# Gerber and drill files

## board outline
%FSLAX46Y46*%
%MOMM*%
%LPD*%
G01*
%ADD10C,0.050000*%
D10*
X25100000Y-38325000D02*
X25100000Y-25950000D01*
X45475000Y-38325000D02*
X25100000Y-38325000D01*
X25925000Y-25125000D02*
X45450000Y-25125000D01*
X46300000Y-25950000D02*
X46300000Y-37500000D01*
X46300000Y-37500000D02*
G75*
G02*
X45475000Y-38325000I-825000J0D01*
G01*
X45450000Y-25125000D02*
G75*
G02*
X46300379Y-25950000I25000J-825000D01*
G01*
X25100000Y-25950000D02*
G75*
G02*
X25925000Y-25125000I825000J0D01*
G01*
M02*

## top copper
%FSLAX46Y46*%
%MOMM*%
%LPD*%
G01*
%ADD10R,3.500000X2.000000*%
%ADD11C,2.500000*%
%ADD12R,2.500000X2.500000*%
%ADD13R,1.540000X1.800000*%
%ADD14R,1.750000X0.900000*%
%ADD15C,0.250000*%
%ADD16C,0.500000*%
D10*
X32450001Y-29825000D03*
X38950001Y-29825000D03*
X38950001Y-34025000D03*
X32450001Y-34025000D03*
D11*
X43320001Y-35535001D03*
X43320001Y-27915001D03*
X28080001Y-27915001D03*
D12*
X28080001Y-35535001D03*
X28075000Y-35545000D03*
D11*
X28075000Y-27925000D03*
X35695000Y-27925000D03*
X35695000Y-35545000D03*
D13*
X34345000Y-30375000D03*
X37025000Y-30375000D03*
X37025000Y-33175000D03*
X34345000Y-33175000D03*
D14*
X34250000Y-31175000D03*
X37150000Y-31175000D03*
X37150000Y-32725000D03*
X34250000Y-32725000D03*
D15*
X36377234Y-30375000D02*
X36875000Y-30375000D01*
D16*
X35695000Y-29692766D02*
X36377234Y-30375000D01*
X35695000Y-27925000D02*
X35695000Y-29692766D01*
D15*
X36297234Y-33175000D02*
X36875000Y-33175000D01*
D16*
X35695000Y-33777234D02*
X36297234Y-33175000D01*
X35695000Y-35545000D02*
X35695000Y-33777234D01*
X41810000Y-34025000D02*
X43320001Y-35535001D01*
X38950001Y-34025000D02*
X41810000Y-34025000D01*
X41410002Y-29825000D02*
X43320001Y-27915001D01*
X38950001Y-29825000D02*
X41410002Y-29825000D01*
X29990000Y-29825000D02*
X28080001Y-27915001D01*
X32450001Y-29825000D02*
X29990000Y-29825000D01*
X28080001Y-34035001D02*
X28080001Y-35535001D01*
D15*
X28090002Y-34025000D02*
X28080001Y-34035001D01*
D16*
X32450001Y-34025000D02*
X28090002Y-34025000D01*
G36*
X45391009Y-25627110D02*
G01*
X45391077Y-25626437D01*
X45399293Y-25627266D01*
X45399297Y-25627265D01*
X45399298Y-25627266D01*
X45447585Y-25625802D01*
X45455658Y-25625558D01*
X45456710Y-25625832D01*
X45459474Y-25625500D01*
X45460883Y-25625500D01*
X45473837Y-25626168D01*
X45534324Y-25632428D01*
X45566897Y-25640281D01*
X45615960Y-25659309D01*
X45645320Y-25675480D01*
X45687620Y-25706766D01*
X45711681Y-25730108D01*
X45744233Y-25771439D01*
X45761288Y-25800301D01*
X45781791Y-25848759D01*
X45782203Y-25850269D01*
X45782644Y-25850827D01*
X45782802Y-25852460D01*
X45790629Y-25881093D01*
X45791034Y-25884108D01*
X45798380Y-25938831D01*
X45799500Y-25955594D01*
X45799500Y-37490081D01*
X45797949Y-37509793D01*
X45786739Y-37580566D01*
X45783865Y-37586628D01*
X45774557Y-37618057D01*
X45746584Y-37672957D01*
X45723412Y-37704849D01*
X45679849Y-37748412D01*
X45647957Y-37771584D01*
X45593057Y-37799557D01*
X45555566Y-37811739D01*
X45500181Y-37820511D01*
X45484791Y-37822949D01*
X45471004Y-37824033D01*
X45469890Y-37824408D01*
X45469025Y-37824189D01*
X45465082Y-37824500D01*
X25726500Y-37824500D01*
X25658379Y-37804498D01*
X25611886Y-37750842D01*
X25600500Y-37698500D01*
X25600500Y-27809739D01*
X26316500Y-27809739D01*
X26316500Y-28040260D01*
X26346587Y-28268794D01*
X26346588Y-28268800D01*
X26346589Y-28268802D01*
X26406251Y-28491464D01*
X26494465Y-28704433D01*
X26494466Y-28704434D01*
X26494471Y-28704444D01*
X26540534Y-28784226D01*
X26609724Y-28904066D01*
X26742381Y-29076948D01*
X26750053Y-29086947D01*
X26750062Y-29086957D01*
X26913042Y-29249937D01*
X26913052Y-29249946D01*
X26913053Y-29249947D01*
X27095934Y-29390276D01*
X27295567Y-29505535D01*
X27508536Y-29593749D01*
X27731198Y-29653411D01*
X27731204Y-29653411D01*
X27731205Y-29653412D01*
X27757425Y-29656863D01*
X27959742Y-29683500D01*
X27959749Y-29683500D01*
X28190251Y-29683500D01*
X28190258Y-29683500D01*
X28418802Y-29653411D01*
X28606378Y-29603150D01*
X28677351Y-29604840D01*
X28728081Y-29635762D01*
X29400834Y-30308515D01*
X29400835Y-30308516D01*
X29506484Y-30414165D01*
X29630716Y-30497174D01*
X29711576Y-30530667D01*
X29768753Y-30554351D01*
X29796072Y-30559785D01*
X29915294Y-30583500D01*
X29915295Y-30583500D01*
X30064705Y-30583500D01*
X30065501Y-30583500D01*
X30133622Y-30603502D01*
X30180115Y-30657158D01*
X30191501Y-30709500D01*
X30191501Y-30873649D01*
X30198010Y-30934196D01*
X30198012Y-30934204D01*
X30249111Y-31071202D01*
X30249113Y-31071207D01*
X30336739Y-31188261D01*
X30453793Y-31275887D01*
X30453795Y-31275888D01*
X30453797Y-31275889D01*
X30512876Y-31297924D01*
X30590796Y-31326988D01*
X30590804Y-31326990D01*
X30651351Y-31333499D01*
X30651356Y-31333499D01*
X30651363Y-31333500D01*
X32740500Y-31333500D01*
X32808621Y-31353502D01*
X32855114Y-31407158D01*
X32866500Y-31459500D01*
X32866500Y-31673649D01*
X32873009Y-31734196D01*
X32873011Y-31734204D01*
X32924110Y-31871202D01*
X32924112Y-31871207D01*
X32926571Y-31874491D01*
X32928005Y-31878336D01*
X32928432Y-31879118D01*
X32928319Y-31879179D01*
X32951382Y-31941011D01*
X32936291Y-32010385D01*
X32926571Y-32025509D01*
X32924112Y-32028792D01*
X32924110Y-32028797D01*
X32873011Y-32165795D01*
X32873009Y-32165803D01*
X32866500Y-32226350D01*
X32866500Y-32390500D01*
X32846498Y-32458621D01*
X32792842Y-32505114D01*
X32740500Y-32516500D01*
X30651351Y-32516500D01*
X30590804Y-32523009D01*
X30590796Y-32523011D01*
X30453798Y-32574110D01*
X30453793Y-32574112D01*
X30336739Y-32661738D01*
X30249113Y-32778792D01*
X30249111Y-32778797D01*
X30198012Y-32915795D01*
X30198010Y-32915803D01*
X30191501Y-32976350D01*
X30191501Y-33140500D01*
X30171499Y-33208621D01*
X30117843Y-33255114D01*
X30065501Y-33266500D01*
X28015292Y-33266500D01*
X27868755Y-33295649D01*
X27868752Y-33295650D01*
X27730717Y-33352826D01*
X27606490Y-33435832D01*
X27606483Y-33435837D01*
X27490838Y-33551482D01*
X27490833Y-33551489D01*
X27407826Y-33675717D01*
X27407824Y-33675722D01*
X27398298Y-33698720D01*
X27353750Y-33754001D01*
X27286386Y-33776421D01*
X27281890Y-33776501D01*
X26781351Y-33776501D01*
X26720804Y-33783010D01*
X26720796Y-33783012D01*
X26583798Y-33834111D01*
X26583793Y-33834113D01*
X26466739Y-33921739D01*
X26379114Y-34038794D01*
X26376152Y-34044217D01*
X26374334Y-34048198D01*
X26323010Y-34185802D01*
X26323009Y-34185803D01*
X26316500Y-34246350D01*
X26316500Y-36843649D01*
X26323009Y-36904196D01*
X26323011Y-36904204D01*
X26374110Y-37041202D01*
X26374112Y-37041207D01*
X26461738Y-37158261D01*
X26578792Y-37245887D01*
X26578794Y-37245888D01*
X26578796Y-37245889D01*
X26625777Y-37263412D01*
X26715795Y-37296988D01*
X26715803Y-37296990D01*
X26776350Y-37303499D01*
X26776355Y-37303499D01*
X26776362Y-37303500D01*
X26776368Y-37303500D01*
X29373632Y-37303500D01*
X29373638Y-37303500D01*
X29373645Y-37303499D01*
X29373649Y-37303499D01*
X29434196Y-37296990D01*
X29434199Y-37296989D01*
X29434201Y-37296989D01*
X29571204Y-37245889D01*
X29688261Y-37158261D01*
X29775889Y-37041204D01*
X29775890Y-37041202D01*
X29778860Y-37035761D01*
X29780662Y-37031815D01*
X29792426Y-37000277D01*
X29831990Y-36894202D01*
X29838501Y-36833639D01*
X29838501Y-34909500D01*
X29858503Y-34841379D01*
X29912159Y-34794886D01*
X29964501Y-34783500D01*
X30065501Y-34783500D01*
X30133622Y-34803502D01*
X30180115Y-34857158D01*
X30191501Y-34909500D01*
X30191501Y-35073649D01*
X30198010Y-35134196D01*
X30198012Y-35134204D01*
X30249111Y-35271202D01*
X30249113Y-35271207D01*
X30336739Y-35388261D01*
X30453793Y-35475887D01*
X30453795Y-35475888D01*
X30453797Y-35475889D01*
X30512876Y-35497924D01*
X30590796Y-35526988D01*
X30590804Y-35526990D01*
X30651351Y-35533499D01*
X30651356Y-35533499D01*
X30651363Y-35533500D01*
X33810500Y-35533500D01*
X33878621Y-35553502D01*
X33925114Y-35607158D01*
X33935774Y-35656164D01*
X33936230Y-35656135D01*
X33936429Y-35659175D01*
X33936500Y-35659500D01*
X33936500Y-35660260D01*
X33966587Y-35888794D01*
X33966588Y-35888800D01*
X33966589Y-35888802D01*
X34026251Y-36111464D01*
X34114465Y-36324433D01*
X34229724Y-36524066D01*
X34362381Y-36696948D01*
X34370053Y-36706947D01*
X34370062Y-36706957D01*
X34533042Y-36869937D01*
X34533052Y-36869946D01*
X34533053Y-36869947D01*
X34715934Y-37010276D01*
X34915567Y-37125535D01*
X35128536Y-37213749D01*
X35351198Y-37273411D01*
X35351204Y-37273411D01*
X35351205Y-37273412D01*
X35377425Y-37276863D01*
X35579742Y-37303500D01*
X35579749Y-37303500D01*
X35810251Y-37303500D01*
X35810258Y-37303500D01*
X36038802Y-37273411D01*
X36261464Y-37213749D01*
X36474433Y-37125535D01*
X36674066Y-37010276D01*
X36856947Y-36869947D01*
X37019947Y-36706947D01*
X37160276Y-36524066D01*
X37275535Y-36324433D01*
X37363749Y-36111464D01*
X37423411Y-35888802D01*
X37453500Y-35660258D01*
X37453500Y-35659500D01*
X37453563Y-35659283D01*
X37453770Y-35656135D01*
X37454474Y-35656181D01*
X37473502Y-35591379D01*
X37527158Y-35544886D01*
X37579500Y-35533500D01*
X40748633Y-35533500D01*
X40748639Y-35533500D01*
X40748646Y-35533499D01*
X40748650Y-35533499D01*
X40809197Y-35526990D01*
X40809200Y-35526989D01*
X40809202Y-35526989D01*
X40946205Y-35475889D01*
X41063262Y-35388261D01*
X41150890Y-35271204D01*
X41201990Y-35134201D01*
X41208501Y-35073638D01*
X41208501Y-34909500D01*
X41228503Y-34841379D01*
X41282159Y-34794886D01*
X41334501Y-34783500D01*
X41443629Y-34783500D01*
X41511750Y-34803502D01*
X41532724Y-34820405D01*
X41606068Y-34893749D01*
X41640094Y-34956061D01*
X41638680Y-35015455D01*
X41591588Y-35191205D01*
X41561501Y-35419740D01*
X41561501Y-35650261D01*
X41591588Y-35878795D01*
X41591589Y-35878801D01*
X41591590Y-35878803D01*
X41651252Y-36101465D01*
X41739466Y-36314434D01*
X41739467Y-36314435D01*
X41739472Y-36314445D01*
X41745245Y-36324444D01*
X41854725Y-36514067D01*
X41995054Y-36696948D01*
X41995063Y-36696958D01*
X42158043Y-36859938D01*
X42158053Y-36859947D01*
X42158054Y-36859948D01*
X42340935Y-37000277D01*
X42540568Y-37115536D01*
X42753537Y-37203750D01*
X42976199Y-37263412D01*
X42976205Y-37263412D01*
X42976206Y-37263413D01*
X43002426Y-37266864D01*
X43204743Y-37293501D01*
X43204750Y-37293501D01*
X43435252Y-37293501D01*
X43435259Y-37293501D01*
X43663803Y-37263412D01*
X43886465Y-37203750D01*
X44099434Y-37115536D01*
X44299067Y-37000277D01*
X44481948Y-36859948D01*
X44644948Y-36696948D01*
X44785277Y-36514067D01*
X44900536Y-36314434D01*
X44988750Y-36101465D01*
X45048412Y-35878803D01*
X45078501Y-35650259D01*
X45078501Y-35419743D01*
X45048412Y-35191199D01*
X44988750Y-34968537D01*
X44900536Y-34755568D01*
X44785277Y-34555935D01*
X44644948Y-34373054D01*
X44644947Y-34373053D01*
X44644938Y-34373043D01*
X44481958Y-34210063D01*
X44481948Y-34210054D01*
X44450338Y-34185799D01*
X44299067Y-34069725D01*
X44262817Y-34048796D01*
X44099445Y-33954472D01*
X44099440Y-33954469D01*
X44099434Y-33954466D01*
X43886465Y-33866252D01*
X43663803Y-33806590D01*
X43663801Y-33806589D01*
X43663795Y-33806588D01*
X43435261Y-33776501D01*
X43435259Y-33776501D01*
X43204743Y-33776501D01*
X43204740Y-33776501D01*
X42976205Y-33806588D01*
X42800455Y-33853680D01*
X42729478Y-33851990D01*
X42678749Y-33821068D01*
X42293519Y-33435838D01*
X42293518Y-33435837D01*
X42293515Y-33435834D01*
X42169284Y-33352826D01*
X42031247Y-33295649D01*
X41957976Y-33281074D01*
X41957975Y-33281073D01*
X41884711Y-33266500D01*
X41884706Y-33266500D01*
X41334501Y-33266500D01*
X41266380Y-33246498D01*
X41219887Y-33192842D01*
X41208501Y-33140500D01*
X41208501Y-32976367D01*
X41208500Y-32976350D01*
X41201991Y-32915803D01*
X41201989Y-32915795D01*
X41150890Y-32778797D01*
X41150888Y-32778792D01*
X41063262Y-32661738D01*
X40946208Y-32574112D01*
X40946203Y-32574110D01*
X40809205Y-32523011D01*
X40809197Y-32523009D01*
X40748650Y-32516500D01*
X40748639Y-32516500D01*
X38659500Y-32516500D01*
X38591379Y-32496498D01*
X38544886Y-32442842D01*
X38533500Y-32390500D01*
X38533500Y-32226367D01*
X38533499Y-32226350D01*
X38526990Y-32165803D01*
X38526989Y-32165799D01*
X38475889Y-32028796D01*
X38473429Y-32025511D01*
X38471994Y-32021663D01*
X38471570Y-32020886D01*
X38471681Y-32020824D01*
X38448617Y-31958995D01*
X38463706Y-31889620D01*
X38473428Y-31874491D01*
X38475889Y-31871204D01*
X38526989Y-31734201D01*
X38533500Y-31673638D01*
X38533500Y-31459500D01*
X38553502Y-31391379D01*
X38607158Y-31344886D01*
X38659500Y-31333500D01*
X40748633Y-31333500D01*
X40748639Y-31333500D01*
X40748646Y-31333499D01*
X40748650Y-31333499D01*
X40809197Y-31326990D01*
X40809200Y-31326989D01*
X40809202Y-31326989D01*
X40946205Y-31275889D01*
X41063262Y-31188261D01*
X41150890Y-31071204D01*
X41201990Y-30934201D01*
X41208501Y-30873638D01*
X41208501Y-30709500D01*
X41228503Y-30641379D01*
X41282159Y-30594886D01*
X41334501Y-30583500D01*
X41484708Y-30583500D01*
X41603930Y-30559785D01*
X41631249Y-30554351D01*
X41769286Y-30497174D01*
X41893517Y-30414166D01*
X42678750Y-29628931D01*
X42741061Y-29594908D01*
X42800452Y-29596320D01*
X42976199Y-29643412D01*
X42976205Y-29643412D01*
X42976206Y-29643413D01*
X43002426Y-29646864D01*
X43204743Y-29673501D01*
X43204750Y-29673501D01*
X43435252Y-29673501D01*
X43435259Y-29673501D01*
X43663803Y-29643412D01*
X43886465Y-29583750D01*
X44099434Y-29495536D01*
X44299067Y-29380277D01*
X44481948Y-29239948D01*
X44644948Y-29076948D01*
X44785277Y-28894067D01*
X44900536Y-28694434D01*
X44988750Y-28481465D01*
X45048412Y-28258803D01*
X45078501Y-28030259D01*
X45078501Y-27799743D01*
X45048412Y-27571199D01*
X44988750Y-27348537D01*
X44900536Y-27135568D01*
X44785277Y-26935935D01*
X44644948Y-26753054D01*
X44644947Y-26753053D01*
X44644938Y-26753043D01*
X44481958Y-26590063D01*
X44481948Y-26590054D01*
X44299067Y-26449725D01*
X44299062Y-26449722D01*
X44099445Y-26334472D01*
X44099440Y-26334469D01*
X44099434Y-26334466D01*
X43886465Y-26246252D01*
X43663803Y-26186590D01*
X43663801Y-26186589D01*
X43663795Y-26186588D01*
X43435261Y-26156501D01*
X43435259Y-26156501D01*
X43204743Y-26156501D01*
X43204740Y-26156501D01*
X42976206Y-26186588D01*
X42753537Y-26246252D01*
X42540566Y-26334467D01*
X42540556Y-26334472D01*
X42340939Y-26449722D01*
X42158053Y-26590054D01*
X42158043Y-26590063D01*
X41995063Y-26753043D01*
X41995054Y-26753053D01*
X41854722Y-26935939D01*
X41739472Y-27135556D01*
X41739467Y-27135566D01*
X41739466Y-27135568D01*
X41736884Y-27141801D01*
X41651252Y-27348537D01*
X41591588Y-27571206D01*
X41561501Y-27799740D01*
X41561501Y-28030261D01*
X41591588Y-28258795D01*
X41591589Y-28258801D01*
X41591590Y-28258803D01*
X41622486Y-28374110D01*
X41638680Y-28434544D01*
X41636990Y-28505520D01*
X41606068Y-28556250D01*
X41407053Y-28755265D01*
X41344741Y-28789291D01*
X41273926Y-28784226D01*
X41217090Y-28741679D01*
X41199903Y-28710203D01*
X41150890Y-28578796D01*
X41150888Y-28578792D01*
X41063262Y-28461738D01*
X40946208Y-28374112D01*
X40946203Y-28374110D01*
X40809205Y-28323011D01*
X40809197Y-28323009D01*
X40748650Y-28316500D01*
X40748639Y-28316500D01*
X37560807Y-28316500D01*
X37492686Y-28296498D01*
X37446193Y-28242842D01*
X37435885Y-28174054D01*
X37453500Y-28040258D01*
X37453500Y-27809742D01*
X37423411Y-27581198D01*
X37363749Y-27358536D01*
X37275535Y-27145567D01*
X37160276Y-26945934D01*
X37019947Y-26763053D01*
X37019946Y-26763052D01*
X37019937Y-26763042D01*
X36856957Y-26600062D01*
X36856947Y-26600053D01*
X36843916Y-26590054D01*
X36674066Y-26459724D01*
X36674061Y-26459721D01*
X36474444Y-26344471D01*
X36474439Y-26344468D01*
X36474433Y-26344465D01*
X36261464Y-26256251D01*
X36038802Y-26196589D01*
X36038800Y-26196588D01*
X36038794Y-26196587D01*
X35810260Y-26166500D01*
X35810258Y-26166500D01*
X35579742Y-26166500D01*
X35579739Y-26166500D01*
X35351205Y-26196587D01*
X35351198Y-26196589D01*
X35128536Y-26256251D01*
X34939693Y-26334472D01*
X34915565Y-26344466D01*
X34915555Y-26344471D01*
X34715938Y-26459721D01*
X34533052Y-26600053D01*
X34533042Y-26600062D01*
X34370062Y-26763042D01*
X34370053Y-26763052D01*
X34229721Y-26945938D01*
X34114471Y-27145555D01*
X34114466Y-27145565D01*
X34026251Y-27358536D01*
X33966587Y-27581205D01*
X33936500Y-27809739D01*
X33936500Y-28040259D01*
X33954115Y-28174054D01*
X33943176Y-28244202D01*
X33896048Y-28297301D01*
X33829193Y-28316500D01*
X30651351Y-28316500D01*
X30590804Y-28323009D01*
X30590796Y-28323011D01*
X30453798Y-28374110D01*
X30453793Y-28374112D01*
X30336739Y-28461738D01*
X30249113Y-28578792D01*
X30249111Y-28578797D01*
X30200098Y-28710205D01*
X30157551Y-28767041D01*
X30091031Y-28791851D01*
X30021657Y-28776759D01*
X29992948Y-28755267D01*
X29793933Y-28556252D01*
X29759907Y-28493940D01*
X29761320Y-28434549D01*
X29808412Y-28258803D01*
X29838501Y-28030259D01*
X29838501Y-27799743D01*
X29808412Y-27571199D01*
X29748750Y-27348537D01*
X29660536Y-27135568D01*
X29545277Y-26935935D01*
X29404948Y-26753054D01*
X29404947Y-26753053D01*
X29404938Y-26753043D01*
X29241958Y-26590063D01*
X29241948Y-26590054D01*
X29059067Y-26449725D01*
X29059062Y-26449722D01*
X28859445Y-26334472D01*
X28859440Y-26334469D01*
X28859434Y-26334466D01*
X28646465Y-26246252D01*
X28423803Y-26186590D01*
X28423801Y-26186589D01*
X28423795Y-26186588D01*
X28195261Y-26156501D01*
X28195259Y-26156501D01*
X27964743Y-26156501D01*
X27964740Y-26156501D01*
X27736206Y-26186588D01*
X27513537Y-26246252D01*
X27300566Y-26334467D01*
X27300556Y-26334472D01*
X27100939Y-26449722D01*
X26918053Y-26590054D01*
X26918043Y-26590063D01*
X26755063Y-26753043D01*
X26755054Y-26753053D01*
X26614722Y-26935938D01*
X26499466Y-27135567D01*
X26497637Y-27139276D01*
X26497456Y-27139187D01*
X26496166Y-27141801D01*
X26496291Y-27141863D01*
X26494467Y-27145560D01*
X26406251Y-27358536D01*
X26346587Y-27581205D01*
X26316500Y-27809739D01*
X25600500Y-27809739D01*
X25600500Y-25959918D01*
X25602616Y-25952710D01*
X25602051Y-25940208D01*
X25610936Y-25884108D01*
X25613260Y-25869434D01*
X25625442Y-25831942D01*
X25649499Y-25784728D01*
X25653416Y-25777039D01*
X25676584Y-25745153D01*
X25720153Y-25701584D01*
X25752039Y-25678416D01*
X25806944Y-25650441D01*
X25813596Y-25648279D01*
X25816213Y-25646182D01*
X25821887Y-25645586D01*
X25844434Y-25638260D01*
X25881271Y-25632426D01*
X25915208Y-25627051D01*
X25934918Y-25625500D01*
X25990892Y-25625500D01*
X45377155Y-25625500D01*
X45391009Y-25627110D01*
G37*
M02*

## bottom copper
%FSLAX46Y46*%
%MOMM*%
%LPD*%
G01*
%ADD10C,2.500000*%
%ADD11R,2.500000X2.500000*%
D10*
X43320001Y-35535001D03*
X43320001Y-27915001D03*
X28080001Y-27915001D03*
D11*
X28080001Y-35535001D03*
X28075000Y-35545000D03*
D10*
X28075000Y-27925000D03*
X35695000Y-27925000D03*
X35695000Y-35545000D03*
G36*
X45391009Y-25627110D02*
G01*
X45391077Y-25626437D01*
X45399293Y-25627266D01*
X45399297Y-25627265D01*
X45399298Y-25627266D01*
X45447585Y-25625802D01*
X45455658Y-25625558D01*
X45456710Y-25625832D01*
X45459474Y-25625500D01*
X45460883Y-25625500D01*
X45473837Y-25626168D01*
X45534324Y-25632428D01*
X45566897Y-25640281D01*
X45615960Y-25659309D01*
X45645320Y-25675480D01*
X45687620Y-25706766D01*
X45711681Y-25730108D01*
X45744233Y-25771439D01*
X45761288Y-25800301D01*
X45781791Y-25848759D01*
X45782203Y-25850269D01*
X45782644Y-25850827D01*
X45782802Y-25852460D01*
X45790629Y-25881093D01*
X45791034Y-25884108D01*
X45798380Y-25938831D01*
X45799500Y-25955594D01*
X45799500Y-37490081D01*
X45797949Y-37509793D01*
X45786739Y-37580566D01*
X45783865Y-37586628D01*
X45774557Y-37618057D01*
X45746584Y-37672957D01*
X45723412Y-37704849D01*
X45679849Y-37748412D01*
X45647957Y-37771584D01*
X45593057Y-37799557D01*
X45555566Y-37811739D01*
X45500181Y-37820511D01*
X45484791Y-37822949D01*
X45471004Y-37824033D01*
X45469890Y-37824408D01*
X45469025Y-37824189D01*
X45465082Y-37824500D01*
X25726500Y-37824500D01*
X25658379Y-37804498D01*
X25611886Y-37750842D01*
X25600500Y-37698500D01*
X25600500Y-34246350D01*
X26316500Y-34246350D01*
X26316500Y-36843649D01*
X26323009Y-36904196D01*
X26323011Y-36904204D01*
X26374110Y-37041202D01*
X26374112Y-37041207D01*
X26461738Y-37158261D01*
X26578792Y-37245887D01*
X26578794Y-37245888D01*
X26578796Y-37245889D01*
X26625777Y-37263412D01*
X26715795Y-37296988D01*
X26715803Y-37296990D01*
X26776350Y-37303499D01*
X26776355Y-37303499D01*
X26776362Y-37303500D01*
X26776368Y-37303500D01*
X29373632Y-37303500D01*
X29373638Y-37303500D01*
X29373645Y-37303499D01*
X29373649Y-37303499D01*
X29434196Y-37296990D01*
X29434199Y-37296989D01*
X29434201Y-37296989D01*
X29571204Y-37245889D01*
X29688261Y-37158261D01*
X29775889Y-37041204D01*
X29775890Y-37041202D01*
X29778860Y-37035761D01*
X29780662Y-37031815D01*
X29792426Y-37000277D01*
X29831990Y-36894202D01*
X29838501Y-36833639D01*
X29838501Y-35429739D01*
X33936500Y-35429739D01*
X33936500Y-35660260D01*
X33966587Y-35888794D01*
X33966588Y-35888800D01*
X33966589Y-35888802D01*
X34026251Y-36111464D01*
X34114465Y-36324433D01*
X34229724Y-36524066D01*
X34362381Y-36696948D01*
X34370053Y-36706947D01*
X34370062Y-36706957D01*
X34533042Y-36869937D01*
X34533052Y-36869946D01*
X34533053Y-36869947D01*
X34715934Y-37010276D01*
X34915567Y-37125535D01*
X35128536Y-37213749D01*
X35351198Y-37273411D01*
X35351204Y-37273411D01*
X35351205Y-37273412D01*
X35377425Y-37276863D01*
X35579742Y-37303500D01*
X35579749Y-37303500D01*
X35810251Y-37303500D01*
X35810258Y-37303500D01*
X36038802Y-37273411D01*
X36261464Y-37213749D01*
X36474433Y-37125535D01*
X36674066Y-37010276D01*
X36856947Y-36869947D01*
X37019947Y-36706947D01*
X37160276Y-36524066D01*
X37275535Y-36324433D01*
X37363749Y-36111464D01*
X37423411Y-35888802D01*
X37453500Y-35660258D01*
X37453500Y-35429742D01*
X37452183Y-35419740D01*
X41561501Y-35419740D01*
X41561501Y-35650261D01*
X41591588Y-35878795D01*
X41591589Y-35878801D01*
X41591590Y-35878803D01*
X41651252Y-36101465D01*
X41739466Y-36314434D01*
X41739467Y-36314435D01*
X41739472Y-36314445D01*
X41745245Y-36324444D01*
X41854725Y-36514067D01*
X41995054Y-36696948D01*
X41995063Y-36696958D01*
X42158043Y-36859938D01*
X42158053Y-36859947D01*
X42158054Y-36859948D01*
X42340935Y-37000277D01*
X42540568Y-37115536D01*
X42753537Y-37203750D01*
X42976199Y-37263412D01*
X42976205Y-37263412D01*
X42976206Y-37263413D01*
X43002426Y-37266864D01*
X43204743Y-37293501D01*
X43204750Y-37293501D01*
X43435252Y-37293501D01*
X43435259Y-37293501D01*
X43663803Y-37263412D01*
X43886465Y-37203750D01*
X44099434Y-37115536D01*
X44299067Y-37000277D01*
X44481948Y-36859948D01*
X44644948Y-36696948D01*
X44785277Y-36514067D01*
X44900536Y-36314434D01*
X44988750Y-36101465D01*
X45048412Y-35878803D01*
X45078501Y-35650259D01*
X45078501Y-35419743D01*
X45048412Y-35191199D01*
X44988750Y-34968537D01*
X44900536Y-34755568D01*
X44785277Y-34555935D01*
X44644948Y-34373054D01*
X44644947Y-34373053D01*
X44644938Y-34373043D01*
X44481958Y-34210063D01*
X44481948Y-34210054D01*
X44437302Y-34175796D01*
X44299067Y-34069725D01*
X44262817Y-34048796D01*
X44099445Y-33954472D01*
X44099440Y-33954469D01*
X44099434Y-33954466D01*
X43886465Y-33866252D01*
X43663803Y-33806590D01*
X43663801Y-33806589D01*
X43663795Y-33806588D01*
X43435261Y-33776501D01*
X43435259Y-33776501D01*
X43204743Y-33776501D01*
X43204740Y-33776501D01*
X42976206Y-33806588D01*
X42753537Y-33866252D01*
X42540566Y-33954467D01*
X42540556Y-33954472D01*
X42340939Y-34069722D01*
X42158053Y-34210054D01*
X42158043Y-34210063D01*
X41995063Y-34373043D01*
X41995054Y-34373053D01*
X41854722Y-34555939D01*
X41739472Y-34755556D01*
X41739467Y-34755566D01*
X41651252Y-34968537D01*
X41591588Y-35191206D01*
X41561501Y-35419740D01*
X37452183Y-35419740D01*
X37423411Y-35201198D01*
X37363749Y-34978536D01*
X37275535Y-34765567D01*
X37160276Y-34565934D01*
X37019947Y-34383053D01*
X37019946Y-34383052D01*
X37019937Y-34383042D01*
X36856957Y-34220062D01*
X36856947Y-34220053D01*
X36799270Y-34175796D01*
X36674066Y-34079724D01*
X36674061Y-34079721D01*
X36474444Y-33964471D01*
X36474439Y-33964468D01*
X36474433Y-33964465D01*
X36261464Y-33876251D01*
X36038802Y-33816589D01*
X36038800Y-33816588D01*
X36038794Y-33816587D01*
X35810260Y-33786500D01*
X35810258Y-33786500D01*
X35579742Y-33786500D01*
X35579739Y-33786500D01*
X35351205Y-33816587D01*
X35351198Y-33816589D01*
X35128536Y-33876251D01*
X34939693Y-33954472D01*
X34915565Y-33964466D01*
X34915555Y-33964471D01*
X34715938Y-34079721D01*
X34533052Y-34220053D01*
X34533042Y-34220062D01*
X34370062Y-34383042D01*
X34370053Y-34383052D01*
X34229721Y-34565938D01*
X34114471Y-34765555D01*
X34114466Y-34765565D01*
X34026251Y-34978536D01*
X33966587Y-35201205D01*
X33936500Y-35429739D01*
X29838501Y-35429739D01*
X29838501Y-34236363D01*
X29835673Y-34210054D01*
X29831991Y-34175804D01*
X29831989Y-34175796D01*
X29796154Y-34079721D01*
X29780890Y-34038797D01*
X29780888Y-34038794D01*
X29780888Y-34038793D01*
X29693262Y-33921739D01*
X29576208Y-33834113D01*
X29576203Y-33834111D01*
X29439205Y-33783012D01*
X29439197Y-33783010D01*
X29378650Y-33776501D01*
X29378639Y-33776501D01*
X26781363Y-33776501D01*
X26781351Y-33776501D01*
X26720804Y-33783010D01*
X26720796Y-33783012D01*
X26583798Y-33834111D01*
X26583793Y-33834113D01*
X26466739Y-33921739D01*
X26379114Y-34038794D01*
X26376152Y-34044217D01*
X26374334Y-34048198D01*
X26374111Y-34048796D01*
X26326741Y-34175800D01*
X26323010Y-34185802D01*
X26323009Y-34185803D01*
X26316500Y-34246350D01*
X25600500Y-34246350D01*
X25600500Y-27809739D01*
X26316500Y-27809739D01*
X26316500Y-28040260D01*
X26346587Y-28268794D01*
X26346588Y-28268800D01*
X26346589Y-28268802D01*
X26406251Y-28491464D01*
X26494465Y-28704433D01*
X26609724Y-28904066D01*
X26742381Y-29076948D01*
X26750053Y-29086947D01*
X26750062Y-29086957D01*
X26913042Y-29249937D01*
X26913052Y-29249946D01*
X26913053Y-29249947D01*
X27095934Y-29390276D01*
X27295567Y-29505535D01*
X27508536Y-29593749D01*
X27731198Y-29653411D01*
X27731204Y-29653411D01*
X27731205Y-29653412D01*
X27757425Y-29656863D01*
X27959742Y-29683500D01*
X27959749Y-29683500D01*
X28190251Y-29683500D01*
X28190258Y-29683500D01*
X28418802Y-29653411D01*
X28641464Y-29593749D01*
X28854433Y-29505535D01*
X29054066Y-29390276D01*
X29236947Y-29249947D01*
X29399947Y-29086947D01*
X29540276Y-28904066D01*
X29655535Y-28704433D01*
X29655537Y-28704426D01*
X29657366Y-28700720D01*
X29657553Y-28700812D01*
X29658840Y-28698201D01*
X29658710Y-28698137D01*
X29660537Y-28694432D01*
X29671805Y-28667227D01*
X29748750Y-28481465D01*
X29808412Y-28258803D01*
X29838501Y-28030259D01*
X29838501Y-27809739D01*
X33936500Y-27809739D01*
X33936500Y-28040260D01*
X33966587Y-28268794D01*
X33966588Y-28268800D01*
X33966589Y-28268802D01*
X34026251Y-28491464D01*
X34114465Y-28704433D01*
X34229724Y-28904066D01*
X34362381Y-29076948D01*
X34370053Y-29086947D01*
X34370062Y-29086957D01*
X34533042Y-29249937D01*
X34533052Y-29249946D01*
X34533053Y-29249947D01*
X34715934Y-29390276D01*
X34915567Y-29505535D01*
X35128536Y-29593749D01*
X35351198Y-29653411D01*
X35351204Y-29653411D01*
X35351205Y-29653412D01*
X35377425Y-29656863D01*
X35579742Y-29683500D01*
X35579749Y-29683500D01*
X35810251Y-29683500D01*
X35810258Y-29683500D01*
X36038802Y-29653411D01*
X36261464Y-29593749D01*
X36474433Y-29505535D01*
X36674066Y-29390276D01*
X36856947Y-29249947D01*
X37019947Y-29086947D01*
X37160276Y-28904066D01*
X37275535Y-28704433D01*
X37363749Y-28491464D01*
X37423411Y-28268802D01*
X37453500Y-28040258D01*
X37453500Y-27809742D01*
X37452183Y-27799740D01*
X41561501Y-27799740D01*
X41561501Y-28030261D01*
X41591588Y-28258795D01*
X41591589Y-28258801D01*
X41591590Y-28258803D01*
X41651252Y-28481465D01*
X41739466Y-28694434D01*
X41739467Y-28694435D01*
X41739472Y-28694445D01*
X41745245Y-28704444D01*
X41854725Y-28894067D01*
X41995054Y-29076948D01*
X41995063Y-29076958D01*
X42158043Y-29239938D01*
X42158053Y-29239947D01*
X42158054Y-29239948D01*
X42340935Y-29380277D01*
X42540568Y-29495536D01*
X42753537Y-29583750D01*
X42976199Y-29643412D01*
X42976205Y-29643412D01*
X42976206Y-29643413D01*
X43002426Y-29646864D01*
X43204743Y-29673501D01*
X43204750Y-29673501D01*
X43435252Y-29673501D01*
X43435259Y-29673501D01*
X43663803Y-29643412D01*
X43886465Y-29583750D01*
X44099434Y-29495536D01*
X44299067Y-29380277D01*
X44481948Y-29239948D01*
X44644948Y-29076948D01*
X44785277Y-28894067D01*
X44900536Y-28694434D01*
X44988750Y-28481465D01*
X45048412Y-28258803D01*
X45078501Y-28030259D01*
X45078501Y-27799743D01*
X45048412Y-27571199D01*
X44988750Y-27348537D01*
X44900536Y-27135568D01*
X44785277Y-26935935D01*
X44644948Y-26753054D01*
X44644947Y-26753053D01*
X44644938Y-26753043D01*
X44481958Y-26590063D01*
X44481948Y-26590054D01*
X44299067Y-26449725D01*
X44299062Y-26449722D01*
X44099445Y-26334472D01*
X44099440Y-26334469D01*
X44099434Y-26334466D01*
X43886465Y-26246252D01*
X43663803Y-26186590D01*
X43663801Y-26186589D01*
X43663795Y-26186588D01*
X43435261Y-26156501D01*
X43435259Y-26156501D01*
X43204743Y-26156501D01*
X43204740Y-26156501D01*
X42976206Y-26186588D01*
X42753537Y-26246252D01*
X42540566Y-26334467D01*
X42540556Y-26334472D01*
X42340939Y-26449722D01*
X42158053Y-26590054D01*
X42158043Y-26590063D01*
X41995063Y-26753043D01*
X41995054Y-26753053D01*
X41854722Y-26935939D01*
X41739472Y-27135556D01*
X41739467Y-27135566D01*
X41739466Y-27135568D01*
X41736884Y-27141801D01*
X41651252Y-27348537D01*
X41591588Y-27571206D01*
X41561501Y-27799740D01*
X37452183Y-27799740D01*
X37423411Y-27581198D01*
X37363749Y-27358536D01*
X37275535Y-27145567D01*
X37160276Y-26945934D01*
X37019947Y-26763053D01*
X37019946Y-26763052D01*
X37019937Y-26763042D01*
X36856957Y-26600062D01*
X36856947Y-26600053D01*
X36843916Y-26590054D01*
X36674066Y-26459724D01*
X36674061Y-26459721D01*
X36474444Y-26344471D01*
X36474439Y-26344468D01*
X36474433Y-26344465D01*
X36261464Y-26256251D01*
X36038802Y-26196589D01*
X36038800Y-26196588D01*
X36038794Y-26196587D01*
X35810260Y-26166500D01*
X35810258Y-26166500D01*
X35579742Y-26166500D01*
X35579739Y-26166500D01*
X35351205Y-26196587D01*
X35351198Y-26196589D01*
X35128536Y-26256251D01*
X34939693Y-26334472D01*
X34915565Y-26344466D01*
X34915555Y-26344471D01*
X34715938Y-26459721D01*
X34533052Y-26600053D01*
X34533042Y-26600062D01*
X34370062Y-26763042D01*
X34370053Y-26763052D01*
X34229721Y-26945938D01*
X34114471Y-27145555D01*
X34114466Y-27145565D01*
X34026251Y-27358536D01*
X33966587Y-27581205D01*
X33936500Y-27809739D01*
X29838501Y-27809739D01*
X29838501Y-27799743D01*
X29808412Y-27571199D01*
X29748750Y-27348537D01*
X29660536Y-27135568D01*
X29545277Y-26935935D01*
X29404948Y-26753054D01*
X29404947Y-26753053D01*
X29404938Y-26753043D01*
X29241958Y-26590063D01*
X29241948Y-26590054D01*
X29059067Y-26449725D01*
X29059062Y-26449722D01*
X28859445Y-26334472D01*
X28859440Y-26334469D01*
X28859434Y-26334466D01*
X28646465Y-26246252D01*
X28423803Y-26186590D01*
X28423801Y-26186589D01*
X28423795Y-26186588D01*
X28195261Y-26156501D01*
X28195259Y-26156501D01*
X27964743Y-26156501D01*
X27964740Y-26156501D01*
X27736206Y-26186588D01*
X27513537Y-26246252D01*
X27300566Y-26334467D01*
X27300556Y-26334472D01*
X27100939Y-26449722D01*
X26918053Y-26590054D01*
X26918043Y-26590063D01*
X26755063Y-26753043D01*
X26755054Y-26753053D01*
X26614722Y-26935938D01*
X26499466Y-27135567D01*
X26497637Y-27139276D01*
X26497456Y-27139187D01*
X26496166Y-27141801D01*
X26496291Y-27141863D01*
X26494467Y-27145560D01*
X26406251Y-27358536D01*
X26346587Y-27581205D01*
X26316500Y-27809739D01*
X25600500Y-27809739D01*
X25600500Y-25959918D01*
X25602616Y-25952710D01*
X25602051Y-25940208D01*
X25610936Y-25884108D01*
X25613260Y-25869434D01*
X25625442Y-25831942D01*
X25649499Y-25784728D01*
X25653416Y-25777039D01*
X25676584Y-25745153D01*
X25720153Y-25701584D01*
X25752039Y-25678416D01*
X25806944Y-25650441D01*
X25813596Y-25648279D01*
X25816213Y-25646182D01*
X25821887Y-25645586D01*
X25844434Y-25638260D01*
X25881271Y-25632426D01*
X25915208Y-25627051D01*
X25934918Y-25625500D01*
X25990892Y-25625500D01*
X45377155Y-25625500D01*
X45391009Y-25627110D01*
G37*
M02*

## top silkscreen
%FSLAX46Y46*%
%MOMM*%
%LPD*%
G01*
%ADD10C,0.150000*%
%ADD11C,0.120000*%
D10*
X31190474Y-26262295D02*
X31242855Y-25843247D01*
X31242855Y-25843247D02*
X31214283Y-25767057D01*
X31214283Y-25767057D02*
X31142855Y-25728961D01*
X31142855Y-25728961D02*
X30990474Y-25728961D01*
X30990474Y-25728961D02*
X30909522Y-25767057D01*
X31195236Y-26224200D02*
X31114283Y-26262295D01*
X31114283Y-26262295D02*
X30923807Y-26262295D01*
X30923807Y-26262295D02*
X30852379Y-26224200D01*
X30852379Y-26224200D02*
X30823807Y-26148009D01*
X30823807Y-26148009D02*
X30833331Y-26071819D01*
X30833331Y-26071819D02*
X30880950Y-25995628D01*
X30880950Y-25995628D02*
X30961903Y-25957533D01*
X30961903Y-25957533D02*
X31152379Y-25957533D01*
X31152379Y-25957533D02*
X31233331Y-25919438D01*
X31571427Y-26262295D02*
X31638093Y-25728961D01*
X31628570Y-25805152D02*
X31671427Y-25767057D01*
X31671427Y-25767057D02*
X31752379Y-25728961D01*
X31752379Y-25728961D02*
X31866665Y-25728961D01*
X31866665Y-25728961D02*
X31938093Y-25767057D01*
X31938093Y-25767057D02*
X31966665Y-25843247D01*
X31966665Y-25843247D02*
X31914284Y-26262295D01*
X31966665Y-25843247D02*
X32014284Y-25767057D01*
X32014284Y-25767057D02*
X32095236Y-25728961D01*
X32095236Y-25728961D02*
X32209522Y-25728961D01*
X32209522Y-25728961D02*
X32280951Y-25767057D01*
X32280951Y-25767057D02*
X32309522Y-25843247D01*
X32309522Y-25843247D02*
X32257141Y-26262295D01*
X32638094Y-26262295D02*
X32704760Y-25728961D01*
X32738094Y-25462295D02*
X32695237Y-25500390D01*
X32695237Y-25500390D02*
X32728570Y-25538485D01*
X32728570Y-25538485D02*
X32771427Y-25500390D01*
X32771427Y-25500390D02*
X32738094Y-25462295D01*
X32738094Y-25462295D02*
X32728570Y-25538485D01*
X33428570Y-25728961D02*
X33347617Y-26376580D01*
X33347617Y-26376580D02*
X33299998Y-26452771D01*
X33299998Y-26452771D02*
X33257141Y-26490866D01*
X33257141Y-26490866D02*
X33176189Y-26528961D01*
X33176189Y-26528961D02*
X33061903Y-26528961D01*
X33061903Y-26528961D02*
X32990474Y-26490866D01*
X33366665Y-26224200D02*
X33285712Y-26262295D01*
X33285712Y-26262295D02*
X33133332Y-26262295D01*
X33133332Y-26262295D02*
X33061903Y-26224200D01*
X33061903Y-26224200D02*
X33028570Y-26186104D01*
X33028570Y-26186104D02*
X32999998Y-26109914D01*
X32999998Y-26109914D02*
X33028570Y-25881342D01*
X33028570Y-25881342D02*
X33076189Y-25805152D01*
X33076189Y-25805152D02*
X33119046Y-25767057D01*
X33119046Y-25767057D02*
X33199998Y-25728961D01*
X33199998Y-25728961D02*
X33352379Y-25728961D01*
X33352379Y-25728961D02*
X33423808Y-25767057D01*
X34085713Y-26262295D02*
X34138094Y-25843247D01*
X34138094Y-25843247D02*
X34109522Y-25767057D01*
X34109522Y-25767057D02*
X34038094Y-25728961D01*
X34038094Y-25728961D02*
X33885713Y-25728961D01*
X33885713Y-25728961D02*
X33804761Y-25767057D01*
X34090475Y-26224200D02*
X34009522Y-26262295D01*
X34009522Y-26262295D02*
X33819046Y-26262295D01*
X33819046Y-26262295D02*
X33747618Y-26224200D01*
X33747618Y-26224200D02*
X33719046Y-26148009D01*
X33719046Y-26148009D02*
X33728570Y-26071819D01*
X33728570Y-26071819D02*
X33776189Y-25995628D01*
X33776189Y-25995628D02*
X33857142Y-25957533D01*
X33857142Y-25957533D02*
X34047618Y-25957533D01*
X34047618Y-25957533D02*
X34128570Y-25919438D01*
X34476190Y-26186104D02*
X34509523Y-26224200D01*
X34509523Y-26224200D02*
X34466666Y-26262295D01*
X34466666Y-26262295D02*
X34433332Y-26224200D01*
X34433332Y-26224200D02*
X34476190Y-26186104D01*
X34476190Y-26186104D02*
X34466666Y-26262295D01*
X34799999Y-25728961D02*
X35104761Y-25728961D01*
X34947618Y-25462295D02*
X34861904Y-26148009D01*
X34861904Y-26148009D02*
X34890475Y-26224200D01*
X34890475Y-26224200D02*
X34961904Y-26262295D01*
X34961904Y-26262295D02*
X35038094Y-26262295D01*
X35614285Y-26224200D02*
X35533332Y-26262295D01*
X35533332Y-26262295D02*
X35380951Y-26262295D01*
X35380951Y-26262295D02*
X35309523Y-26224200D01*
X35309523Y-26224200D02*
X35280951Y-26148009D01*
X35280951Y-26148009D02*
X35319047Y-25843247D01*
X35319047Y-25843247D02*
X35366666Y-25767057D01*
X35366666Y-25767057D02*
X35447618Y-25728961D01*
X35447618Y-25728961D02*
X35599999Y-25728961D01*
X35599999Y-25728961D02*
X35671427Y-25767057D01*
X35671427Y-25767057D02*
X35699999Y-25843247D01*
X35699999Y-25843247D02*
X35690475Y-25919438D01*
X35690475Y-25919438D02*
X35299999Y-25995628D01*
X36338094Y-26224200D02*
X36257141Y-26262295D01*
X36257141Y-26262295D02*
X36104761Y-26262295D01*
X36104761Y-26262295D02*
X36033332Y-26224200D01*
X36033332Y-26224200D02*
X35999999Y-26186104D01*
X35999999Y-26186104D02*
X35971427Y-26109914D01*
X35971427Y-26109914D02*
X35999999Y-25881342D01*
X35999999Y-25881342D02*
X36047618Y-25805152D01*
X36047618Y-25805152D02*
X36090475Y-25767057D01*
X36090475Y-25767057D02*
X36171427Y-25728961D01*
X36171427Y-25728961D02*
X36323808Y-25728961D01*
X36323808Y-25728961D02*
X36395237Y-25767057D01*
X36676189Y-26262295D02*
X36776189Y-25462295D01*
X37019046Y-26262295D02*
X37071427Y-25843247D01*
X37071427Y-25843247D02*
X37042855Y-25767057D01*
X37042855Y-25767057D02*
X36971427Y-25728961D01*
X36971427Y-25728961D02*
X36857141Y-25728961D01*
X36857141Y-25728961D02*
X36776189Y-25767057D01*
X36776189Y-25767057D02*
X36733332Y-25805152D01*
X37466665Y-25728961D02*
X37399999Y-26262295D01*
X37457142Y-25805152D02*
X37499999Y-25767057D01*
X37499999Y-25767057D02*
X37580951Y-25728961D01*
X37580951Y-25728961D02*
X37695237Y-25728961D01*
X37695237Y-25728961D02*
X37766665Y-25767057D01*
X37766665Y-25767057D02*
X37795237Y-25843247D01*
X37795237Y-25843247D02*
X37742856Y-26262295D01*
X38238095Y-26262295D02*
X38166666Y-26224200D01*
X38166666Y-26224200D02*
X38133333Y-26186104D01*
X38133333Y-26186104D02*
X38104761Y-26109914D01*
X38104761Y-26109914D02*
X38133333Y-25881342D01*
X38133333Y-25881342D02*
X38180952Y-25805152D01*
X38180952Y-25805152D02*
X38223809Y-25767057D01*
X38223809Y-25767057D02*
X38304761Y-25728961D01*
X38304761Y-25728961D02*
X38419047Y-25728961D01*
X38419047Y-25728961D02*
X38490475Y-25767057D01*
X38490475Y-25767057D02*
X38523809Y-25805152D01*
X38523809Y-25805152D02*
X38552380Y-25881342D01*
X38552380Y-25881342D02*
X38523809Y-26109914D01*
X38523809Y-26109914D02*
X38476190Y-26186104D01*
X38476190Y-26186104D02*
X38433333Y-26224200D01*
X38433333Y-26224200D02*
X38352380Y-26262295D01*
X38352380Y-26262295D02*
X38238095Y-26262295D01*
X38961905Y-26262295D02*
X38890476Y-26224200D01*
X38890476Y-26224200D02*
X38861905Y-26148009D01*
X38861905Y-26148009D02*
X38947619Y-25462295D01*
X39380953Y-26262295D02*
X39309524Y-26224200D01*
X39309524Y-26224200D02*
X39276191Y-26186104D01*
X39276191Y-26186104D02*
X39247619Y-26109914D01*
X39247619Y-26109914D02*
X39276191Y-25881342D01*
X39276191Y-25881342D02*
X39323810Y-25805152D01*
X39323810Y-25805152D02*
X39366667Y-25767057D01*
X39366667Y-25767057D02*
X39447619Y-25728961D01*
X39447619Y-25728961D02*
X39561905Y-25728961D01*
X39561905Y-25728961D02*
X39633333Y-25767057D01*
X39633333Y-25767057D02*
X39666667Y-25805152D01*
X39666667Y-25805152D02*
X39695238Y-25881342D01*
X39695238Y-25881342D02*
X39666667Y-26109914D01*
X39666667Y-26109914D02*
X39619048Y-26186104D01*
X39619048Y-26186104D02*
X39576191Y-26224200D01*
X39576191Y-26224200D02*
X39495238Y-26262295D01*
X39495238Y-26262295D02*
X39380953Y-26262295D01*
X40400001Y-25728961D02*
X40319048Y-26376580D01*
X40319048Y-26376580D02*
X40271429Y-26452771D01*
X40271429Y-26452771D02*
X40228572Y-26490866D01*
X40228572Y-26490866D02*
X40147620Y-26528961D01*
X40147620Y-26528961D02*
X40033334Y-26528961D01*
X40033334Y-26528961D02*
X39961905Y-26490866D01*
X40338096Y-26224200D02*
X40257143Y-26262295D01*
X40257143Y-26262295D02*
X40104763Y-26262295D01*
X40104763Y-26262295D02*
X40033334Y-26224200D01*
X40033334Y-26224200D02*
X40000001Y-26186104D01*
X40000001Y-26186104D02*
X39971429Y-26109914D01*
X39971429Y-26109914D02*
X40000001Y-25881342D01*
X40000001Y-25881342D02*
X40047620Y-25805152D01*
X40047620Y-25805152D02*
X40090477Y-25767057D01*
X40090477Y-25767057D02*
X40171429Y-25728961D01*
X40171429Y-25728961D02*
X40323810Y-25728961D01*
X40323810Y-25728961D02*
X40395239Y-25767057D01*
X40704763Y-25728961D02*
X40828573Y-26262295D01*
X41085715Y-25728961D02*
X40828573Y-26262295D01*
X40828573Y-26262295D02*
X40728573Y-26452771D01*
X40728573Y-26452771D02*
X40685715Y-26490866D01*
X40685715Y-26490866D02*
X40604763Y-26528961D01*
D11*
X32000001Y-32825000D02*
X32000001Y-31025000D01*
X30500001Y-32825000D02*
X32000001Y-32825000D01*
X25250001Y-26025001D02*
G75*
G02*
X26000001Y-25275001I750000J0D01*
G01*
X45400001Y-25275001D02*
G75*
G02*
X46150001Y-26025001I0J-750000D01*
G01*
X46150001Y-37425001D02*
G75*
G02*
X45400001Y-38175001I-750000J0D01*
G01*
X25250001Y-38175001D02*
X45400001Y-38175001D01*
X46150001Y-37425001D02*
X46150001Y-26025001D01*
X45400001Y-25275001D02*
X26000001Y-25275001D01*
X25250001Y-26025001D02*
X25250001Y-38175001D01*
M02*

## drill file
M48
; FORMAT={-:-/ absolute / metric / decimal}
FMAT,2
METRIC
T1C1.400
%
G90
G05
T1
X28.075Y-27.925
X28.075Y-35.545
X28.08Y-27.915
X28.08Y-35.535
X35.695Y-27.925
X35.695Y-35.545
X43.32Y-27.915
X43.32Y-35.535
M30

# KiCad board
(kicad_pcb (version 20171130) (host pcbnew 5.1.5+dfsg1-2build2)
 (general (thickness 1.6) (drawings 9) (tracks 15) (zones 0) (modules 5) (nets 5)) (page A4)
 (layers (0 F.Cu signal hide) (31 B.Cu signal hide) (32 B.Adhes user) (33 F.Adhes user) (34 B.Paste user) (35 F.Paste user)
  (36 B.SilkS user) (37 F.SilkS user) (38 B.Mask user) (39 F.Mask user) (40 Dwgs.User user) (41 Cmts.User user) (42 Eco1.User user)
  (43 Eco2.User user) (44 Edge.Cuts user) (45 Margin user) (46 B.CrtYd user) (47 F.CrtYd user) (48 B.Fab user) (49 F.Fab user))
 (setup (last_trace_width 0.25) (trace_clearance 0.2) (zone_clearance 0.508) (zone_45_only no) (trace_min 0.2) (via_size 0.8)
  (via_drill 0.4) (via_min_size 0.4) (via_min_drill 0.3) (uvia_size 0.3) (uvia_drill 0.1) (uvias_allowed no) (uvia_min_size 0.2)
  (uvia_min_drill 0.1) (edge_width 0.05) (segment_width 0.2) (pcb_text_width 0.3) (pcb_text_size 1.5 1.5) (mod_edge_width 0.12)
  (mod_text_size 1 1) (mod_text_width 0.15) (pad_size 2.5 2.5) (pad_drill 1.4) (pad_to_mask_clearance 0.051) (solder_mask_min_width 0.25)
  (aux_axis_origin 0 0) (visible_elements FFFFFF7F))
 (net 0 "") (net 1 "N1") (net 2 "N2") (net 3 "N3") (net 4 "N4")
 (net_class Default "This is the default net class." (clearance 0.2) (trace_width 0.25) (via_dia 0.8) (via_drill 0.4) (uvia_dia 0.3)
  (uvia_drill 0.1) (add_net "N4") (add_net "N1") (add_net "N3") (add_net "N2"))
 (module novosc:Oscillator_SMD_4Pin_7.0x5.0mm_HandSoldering (layer F.Cu) (at 35.700001 31.925)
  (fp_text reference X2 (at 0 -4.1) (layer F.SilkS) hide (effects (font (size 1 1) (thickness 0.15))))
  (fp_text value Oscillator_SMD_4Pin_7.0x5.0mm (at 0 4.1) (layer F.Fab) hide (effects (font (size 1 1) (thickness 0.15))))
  (fp_line (start -3.7 0.9) (end -3.7 -0.9) (layer F.SilkS) (width 0.12))
  (fp_line (start -5.2 0.9) (end -3.7 0.9) (layer F.SilkS) (width 0.12))
  (pad 4 smd rect (at -3.25 -2.1) (size 3.5 2) (layers F.Cu F.Paste F.Mask) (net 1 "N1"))
  (pad 3 smd rect (at 3.25 -2.1) (size 3.5 2) (layers F.Cu F.Paste F.Mask) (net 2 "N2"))
  (pad 2 smd rect (at 3.25 2.1) (size 3.5 2) (layers F.Cu F.Paste F.Mask) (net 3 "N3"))
  (pad 1 smd rect (at -3.25 2.1) (size 3.5 2) (layers F.Cu F.Paste F.Mask) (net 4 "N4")))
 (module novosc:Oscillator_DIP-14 (layer F.Cu) (at 28.080001 35.535001)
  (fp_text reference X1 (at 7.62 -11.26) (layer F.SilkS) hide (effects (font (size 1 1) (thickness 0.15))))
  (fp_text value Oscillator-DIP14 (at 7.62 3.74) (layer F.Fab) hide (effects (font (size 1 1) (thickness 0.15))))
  (fp_arc (start -2.08 -9.51) (end -2.83 -9.51) (angle 90) (layer F.SilkS) (width 0.12))
  (fp_arc (start 17.32 -9.51) (end 17.32 -10.26) (angle 90) (layer F.SilkS) (width 0.12))
  (fp_arc (start 17.32 1.89) (end 18.07 1.89) (angle 90) (layer F.SilkS) (width 0.12))
  (fp_line (start -2.83 2.64) (end 17.32 2.64) (layer F.SilkS) (width 0.12))
  (fp_line (start 18.07 1.89) (end 18.07 -9.51) (layer F.SilkS) (width 0.12))
  (fp_line (start 17.32 -10.26) (end -2.08 -10.26) (layer F.SilkS) (width 0.12))
  (fp_line (start -2.83 -9.51) (end -2.83 2.64) (layer F.SilkS) (width 0.12))
  (pad 7 thru_hole circle (at 15.24 0) (size 2.5 2.5) (drill 1.4) (layers *.Cu *.Mask) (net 3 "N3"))
  (pad 8 thru_hole circle (at 15.24 -7.62) (size 2.5 2.5) (drill 1.4) (layers *.Cu *.Mask) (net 2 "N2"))
  (pad 14 thru_hole circle (at 0 -7.62) (size 2.5 2.5) (drill 1.4) (layers *.Cu *.Mask) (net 1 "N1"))
  (pad 1 thru_hole rect (at 0 0) (size 2.5 2.5) (drill 1.4) (layers *.Cu *.Mask) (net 4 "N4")))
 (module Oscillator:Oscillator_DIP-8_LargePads (layer F.Cu) (at 28.075 35.545)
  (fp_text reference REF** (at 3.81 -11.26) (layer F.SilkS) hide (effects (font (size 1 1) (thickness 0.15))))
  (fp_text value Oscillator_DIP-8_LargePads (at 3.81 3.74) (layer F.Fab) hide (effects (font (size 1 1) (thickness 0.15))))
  (pad 1 thru_hole rect (at 0 0) (size 2.5 2.5) (drill 1.4) (layers *.Cu *.Mask))
  (pad 8 thru_hole circle (at 0 -7.62) (size 2.5 2.5) (drill 1.4) (layers *.Cu *.Mask))
  (pad 5 thru_hole circle (at 7.62 -7.62) (size 2.5 2.5) (drill 1.4) (layers *.Cu *.Mask))
  (pad 4 thru_hole circle (at 7.62 0) (size 2.5 2.5) (drill 1.4) (layers *.Cu *.Mask)))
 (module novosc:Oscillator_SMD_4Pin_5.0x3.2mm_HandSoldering (layer F.Cu) (at 35.685 31.775)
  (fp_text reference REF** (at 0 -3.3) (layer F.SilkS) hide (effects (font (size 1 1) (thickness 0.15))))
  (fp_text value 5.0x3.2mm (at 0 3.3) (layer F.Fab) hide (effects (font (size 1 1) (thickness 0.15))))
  (pad 4 smd rect (at -1.34 -1.4) (size 1.54 1.8) (layers F.Cu F.Paste F.Mask))
  (pad 3 smd rect (at 1.34 -1.4) (size 1.54 1.8) (layers F.Cu F.Paste F.Mask))
  (pad 2 smd rect (at 1.34 1.4) (size 1.54 1.8) (layers F.Cu F.Paste F.Mask))
  (pad 1 smd rect (at -1.34 1.4) (size 1.54 1.8) (layers F.Cu F.Paste F.Mask)))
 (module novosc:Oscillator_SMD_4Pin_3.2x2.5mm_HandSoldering (layer F.Cu) (at 35.7 31.95)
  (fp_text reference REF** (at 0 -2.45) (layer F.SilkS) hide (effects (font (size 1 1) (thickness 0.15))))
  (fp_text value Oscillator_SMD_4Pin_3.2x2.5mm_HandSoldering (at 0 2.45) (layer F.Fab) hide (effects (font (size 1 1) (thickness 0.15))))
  (pad 4 smd rect (at -1.45 -0.775) (size 1.75 0.9) (layers F.Cu F.Paste F.Mask))
  (pad 3 smd rect (at 1.45 -0.775) (size 1.75 0.9) (layers F.Cu F.Paste F.Mask))
  (pad 2 smd rect (at 1.45 0.775) (size 1.75 0.9) (layers F.Cu F.Paste F.Mask))
  (pad 1 smd rect (at -1.45 0.775) (size 1.75 0.9) (layers F.Cu F.Paste F.Mask)))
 (gr_line (start 25.1 38.325) (end 25.1 25.95) (layer Edge.Cuts) (width 0.05))
 (gr_line (start 45.475 38.325) (end 25.1 38.325) (layer Edge.Cuts) (width 0.05))
 (gr_line (start 25.925 25.125) (end 45.45 25.125) (layer Edge.Cuts) (width 0.05))
 (gr_line (start 46.3 25.95) (end 46.3 37.5) (layer Edge.Cuts) (width 0.05))
 (gr_arc (start 45.475 37.5) (end 46.3 37.5) (angle 90) (layer Edge.Cuts) (width 0.05))
 (gr_arc (start 45.475 25.95) (end 45.45 25.125) (angle 91.73570459) (layer Edge.Cuts) (width 0.05))
 (gr_arc (start 25.925 25.95) (end 25.1 25.95) (angle 90) (layer Edge.Cuts) (width 0.05))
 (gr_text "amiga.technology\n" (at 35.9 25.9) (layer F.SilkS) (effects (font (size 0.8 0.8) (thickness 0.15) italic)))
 (segment (start 36.377234 30.375) (end 36.875 30.375) (width 0.25) (layer F.Cu) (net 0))
 (segment (start 35.695 29.692766) (end 36.377234 30.375) (width 0.5) (layer F.Cu) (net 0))
 (segment (start 35.695 27.925) (end 35.695 29.692766) (width 0.5) (layer F.Cu) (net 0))
 (segment (start 36.297234 33.175) (end 36.875 33.175) (width 0.25) (layer F.Cu) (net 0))
 (segment (start 35.695 33.777234) (end 36.297234 33.175) (width 0.5) (layer F.Cu) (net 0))
 (segment (start 35.695 35.545) (end 35.695 33.777234) (width 0.5) (layer F.Cu) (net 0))
 (segment (start 41.81 34.025) (end 43.320001 35.535001) (width 0.5) (layer F.Cu) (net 3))
 (segment (start 38.950001 34.025) (end 41.81 34.025) (width 0.5) (layer F.Cu) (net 3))
 (segment (start 41.410002 29.825) (end 43.320001 27.915001) (width 0.5) (layer F.Cu) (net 2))
 (segment (start 38.950001 29.825) (end 41.410002 29.825) (width 0.5) (layer F.Cu) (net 2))
 (segment (start 29.99 29.825) (end 28.080001 27.915001) (width 0.5) (layer F.Cu) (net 1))
 (segment (start 32.450001 29.825) (end 29.99 29.825) (width 0.5) (layer F.Cu) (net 1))
 (segment (start 28.080001 34.035001) (end 28.080001 35.535001) (width 0.5) (layer F.Cu) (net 4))
 (segment (start 28.090002 34.025) (end 28.080001 34.035001) (width 0.25) (layer F.Cu) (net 4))
 (segment (start 32.450001 34.025) (end 28.090002 34.025) (width 0.5) (layer F.Cu) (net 4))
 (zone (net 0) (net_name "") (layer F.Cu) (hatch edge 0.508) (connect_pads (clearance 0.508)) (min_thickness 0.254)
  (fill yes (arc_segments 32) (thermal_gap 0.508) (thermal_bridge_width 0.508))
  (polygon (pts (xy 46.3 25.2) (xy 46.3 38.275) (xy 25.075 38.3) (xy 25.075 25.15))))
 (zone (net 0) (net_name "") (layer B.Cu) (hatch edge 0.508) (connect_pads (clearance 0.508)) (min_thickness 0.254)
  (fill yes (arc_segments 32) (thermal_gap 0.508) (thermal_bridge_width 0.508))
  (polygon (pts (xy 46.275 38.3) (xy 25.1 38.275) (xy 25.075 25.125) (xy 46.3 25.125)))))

